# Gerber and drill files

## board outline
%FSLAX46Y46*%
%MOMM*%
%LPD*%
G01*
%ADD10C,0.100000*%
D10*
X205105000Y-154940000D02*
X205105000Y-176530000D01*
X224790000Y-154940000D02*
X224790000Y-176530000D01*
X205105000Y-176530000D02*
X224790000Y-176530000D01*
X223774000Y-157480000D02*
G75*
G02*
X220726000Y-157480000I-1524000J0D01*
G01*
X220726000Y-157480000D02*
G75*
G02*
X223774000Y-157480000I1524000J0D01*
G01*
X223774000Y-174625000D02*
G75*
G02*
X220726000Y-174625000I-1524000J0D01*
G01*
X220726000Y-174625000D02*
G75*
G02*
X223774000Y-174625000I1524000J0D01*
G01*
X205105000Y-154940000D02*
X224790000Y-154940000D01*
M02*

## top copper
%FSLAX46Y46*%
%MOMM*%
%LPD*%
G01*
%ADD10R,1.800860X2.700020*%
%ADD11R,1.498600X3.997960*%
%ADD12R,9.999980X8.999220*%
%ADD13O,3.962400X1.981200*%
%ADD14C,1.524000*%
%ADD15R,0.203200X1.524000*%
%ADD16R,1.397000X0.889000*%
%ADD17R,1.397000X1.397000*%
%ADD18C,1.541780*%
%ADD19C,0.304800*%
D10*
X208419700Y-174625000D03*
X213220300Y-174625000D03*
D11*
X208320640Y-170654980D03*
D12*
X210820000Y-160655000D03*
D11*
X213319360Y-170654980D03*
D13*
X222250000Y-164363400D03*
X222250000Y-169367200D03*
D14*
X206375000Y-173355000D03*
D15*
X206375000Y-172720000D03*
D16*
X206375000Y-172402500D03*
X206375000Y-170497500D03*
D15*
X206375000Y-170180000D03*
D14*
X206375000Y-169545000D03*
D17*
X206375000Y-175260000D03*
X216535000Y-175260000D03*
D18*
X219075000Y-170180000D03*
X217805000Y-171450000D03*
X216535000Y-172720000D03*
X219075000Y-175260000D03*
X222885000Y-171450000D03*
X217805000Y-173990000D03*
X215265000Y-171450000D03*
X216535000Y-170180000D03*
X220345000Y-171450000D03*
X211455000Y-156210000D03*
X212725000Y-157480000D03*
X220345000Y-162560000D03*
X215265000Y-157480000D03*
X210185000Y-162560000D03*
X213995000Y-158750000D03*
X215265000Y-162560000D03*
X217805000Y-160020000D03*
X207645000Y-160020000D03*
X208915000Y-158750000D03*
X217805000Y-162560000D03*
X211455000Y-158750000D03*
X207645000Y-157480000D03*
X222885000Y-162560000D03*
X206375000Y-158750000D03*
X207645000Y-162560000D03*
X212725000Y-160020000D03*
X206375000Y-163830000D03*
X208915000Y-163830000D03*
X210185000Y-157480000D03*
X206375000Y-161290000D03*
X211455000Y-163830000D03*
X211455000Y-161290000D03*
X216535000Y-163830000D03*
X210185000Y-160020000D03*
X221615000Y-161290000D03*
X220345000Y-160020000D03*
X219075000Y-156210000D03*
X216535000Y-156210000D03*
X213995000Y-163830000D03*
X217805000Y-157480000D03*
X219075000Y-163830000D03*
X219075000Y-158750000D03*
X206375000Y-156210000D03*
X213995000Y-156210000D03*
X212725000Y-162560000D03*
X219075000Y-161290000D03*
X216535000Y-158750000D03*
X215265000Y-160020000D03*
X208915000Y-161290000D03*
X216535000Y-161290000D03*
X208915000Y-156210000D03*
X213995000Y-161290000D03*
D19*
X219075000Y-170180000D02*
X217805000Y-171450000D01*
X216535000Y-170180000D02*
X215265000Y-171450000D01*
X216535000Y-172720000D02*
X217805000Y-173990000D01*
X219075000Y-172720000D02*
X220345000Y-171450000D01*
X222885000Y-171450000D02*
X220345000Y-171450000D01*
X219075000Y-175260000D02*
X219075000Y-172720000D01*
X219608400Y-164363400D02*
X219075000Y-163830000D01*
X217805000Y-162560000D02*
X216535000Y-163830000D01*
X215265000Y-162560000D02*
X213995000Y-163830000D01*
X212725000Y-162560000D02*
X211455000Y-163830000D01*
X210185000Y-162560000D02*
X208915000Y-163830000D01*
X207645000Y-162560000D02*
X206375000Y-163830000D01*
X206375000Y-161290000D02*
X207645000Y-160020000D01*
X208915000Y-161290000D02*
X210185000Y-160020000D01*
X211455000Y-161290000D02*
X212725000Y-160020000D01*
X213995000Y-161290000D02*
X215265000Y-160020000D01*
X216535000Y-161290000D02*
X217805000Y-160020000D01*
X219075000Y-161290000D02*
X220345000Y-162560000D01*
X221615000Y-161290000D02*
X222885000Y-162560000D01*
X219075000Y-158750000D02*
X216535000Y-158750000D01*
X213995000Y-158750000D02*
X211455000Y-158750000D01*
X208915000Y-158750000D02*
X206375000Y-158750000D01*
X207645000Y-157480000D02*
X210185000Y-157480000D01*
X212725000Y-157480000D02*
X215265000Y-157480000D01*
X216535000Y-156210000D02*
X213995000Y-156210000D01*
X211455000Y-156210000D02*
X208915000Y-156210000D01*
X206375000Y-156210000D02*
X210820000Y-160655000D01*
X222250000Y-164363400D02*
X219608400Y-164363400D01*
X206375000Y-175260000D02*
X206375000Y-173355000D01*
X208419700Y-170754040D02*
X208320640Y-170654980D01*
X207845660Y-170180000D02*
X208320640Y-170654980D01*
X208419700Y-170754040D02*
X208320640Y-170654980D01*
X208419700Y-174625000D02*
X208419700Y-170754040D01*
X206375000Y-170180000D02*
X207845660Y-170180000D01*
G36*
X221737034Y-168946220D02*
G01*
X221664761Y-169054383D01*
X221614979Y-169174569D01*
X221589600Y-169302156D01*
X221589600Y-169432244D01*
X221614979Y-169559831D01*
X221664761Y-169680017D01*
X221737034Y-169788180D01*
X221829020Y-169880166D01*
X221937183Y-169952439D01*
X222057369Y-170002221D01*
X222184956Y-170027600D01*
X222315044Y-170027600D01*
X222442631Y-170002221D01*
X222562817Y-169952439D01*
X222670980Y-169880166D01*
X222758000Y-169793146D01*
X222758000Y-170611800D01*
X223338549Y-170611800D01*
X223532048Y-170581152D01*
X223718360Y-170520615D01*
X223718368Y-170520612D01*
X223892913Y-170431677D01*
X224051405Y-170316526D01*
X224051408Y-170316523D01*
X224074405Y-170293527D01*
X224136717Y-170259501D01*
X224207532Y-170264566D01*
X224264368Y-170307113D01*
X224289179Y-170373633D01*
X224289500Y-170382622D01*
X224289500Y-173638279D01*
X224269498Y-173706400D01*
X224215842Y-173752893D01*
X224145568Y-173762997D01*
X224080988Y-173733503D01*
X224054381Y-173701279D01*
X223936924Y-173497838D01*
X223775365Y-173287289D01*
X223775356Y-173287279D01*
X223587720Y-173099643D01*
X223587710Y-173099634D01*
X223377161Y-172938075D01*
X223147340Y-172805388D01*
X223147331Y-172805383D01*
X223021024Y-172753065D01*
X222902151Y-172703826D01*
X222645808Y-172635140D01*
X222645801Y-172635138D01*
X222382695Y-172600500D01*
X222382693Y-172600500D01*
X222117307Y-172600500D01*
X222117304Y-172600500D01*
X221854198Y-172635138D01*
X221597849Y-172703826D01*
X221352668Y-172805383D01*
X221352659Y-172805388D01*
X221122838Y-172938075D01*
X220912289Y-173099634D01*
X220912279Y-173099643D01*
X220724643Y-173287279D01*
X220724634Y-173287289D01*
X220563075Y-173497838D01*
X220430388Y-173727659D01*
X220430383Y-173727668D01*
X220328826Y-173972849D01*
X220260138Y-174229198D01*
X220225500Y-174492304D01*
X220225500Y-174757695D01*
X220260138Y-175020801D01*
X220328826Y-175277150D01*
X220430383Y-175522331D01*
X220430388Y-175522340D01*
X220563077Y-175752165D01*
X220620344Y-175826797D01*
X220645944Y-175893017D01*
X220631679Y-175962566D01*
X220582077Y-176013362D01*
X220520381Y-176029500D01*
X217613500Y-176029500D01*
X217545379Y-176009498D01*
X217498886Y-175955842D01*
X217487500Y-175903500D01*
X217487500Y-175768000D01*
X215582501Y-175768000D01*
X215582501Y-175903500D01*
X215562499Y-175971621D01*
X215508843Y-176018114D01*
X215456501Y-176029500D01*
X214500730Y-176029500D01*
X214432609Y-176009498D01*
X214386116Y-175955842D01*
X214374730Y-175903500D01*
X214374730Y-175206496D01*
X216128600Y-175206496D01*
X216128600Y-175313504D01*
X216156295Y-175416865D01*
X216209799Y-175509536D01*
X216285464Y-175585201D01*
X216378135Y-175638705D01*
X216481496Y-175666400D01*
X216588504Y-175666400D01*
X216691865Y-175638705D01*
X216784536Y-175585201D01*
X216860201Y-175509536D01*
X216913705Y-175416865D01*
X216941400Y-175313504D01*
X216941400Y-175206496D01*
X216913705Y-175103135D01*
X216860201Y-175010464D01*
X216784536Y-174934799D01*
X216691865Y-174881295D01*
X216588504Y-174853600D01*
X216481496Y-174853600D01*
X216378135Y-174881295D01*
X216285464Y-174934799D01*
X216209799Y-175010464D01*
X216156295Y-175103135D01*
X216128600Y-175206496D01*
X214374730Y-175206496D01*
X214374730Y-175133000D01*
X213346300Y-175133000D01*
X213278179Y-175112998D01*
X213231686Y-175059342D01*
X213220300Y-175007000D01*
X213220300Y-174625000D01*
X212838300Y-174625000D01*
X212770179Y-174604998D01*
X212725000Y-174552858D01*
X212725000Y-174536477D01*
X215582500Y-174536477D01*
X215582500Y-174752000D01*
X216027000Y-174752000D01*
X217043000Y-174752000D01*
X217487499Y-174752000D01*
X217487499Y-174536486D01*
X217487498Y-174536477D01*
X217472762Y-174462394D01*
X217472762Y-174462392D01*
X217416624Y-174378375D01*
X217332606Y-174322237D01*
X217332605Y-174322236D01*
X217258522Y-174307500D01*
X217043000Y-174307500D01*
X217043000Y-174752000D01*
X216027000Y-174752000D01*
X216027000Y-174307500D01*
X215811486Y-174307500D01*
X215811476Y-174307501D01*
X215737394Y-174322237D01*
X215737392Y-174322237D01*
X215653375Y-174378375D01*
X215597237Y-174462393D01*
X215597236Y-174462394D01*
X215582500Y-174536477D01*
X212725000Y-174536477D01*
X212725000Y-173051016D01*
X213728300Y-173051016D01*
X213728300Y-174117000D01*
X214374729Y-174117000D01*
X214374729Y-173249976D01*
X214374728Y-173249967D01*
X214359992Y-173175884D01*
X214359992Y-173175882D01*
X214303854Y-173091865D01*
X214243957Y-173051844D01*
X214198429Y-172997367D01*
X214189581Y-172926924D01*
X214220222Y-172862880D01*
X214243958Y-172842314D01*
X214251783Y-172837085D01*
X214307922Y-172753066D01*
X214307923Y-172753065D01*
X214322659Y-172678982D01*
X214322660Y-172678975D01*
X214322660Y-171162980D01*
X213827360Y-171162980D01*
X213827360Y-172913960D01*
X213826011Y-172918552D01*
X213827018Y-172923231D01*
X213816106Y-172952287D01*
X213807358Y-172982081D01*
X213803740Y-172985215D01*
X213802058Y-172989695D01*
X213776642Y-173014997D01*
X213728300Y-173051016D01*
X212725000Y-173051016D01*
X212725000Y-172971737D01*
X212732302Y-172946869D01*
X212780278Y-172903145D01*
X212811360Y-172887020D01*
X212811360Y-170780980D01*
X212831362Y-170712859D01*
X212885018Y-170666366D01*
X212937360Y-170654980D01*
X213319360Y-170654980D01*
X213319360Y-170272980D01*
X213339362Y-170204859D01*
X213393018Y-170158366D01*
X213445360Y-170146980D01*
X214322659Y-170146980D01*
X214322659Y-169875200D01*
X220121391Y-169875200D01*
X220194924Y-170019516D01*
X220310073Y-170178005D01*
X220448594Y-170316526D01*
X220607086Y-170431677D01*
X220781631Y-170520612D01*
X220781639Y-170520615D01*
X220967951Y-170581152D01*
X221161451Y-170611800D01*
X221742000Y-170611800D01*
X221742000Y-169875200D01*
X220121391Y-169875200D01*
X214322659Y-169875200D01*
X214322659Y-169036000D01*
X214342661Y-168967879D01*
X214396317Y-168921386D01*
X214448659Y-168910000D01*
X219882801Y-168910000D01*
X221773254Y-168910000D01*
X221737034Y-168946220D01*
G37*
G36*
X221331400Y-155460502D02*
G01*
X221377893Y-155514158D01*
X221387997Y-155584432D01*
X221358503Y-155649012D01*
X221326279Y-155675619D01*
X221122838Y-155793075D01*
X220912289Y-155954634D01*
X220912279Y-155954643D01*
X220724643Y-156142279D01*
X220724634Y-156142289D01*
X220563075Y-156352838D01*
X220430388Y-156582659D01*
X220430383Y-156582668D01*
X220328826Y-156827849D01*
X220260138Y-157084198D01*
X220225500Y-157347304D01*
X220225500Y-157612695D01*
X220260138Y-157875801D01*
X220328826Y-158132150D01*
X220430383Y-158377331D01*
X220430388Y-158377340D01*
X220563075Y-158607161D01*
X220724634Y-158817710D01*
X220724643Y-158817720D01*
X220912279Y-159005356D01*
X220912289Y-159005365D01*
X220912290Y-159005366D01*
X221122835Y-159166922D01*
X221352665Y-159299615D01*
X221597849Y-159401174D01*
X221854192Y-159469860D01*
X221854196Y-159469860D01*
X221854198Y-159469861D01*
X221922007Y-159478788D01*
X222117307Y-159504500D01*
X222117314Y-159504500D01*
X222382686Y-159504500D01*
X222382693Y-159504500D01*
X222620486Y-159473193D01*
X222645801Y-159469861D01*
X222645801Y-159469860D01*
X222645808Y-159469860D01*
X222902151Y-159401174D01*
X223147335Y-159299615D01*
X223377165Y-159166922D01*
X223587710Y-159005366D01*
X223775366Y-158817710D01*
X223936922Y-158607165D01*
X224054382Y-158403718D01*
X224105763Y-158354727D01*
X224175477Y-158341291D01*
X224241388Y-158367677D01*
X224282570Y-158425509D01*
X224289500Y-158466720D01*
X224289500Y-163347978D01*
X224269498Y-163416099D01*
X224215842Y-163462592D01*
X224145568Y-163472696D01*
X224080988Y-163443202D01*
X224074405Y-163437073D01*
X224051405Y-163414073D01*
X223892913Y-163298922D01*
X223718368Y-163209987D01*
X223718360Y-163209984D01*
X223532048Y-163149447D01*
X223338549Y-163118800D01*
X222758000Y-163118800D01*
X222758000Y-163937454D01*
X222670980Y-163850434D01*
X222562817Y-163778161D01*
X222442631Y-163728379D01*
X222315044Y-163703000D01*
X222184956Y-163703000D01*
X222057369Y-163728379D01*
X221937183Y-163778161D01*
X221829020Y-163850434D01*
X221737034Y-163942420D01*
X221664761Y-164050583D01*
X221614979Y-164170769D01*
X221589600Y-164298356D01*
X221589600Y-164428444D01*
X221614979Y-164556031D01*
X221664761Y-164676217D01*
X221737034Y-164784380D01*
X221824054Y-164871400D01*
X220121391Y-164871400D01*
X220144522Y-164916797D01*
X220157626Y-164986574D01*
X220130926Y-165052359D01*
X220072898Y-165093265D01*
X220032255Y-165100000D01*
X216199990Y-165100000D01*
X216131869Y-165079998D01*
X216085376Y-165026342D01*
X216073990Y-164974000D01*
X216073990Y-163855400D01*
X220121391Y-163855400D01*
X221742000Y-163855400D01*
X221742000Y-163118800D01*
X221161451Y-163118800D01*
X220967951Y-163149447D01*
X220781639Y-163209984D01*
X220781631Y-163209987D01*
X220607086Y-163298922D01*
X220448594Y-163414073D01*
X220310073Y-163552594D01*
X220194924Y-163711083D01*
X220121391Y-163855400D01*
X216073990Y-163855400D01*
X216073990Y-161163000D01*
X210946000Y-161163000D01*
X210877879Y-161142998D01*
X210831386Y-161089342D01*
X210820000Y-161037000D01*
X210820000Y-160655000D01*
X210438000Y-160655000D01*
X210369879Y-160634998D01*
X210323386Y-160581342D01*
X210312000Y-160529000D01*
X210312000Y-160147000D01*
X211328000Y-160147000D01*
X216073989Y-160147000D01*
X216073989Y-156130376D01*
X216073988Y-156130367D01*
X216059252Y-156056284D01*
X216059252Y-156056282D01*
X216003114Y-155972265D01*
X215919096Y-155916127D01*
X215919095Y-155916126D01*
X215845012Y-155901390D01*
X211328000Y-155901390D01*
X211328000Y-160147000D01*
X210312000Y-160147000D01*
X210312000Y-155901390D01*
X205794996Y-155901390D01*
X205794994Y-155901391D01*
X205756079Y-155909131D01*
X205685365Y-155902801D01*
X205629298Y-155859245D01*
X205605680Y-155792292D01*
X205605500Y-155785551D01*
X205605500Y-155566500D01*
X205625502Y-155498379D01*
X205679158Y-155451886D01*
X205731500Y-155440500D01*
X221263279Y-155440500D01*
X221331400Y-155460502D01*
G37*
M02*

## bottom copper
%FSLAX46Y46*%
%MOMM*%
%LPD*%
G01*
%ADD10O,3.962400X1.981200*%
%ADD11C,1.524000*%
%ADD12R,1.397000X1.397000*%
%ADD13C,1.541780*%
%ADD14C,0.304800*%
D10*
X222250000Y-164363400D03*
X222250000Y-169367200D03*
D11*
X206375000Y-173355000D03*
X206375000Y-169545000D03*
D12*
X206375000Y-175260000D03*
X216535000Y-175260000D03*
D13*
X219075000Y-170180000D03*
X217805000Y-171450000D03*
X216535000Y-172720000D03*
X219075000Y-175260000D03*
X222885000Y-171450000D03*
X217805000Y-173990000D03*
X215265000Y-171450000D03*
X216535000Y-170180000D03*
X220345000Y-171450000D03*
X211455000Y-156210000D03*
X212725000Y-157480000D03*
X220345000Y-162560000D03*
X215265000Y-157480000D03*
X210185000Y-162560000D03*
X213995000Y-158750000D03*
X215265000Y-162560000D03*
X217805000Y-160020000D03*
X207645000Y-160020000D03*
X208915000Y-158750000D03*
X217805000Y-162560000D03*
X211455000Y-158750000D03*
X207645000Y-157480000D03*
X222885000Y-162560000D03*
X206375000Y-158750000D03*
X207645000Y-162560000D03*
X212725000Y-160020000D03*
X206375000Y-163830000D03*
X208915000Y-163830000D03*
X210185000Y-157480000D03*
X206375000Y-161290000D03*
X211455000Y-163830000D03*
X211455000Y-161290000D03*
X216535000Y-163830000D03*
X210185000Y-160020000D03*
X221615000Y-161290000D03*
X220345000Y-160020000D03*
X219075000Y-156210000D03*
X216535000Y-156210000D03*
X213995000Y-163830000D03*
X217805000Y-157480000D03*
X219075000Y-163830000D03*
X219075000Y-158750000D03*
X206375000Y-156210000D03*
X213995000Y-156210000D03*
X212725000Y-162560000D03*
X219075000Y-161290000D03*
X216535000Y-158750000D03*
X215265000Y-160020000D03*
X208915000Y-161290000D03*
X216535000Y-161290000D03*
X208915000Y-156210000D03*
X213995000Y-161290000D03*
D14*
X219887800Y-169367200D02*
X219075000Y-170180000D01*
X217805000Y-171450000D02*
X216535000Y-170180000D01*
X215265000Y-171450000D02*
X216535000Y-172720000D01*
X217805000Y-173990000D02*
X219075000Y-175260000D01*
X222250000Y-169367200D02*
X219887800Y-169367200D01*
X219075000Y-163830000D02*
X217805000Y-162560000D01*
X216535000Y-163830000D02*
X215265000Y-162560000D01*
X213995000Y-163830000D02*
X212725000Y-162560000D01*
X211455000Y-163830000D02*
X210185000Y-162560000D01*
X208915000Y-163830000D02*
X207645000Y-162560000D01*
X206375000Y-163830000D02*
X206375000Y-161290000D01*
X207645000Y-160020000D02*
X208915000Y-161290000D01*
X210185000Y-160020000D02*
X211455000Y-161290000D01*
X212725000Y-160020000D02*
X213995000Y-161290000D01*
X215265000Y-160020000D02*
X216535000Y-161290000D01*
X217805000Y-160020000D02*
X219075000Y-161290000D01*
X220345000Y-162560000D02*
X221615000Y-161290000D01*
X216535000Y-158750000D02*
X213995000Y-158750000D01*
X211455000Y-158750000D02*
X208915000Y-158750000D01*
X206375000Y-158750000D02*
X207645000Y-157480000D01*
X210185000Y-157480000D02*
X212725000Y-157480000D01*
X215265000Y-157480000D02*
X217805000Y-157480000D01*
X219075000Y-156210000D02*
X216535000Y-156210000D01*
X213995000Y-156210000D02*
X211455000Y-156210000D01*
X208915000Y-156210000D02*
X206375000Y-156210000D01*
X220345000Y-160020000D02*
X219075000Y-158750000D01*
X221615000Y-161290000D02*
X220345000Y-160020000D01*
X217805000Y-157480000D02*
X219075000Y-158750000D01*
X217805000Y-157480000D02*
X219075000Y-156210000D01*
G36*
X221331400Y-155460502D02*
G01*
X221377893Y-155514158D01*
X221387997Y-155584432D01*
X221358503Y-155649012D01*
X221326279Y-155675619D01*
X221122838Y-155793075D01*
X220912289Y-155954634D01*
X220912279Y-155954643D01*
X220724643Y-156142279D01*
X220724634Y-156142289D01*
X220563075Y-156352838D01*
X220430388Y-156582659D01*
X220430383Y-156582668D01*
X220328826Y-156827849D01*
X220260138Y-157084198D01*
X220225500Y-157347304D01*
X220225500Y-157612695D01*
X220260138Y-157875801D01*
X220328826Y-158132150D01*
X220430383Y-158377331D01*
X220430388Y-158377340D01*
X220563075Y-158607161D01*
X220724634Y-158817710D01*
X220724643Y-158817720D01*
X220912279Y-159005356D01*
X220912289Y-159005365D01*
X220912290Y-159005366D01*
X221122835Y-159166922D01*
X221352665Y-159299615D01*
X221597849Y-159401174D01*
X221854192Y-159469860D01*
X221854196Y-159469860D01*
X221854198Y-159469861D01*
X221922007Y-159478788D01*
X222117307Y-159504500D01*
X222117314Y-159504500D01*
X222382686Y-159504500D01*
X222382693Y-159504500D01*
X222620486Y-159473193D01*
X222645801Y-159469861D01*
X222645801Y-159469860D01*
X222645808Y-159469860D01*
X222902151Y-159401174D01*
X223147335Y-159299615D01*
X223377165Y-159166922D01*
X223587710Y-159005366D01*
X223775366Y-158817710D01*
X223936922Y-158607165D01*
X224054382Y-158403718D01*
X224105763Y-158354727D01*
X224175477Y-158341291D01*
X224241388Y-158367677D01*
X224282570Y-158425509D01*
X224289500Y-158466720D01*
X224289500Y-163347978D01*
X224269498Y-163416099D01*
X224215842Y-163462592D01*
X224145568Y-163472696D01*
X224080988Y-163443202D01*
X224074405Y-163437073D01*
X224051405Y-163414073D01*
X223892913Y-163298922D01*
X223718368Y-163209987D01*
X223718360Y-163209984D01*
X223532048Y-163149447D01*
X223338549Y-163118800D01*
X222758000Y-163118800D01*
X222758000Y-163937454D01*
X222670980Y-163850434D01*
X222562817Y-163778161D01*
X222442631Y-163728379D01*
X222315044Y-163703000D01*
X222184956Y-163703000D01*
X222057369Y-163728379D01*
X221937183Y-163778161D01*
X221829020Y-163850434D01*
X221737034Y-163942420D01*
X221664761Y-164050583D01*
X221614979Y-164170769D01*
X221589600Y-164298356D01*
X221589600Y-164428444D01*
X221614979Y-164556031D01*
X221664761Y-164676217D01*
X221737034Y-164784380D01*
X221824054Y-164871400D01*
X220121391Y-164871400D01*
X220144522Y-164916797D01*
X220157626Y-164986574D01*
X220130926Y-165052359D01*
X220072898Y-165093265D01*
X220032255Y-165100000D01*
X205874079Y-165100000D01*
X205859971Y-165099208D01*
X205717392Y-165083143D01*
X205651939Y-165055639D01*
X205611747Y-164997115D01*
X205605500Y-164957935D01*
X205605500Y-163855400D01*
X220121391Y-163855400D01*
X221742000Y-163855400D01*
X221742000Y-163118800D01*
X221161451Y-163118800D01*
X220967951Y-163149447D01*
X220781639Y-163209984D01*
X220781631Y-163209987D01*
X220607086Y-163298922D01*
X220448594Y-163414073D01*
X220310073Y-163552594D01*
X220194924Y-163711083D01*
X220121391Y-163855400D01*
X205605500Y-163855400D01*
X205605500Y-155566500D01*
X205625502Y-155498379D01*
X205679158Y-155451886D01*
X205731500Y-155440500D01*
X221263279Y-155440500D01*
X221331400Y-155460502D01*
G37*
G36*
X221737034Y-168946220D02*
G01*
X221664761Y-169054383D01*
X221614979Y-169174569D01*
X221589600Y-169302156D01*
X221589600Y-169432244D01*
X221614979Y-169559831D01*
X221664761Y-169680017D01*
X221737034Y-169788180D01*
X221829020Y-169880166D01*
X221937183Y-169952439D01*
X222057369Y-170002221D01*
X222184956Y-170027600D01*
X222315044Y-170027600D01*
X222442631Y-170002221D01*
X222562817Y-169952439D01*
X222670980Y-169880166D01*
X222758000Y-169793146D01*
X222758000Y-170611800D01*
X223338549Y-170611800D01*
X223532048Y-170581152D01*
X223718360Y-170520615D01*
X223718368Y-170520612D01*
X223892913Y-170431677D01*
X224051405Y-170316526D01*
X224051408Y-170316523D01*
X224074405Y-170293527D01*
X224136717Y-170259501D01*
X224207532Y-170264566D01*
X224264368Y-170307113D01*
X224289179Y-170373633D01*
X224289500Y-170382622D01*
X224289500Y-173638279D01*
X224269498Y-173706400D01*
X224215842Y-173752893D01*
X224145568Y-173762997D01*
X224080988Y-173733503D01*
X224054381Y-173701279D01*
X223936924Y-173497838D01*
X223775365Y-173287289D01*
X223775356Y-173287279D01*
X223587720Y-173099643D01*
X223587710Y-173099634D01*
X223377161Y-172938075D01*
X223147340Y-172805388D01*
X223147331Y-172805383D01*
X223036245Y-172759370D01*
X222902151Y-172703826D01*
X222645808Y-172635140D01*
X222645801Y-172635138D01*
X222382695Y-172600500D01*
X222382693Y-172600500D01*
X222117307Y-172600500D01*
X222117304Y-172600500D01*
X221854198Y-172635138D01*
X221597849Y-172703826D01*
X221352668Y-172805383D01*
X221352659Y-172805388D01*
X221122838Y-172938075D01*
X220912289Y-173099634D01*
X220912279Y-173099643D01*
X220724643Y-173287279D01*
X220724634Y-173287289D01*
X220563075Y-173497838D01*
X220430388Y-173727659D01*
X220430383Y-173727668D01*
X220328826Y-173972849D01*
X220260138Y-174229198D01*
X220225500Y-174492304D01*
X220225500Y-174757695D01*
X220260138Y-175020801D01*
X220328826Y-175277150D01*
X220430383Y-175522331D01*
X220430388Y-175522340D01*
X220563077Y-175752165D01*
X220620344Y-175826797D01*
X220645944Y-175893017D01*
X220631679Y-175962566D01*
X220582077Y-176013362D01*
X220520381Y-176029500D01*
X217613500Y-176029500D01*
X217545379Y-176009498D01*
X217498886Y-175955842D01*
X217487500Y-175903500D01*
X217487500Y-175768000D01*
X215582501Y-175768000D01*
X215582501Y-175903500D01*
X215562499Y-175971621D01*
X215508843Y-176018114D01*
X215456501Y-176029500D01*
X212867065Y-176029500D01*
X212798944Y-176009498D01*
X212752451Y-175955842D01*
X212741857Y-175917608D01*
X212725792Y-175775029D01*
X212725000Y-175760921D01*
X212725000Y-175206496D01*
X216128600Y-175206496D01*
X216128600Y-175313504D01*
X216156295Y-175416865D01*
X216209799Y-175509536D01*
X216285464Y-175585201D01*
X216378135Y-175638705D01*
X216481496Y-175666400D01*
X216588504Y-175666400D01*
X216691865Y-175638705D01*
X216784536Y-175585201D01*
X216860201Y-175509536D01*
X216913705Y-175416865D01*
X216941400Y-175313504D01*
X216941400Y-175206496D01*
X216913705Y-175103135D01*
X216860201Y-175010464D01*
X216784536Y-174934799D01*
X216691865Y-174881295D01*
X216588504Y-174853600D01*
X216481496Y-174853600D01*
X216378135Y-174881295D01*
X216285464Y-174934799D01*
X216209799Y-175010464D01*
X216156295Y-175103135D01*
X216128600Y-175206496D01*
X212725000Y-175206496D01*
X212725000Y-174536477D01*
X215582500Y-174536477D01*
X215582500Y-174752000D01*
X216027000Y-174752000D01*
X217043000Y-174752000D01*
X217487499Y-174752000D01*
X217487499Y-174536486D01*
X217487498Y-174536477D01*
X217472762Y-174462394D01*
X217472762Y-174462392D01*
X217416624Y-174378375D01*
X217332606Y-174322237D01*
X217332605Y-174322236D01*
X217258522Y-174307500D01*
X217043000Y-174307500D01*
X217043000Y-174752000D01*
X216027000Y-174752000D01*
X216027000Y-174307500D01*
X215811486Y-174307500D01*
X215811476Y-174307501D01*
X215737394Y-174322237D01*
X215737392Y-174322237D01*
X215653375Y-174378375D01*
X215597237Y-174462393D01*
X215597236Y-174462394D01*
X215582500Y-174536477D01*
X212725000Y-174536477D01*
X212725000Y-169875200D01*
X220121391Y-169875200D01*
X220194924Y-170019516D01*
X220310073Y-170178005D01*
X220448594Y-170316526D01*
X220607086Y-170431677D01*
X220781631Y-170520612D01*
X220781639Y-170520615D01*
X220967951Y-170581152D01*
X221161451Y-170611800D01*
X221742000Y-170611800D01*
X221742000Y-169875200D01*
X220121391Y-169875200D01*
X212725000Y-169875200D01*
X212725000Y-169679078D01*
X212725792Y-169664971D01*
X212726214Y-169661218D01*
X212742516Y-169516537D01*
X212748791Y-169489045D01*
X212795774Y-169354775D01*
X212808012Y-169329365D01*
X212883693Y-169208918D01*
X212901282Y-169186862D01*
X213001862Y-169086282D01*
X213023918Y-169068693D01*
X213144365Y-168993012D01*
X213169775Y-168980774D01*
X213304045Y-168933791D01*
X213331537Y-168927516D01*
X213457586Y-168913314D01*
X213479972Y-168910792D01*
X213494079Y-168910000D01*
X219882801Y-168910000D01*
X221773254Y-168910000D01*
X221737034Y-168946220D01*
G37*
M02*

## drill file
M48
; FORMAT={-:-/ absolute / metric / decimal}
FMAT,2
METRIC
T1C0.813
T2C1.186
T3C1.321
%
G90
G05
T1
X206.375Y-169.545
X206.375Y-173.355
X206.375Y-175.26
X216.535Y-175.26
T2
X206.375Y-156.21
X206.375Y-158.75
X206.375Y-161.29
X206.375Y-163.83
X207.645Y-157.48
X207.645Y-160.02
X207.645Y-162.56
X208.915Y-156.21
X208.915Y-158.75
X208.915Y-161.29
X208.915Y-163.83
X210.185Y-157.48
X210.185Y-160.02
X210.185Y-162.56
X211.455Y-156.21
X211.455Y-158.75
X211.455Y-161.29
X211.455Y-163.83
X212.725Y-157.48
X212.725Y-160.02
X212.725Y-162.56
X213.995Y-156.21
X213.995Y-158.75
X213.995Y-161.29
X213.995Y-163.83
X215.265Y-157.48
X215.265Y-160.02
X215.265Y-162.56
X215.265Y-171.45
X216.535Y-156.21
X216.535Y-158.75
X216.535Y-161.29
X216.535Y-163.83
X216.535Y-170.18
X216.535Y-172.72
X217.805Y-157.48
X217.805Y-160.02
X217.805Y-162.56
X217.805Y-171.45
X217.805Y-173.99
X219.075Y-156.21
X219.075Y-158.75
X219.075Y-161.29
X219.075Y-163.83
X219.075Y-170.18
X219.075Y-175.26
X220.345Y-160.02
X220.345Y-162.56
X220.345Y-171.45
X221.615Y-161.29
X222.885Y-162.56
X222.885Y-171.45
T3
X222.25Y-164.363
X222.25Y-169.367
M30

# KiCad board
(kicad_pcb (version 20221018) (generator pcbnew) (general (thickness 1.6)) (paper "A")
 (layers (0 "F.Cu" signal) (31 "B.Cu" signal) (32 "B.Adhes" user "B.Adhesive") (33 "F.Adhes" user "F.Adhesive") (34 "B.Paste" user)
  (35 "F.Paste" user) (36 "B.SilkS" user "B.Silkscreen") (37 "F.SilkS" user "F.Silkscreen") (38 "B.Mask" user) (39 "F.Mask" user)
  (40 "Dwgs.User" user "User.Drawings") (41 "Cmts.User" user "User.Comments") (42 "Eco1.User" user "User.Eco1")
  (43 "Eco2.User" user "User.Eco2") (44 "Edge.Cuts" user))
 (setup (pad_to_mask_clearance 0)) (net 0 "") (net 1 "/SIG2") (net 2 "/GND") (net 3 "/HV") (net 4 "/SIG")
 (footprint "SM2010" (layer "F.Cu") (at 210.82 174.625)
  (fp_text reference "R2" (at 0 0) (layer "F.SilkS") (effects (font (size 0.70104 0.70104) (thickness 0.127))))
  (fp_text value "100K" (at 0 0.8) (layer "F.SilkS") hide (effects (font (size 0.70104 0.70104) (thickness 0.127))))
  (pad "1" smd rect (at -2.4003 0) (size 1.80086 2.70002) (layers "F.Cu" "F.Paste" "F.Mask") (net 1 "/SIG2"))
  (pad "2" smd rect (at 2.4003 0) (size 1.80086 2.70002) (layers "F.Cu" "F.Paste" "F.Mask") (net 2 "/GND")))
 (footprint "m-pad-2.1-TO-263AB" (layer "F.Cu") (at 210.82 160.655)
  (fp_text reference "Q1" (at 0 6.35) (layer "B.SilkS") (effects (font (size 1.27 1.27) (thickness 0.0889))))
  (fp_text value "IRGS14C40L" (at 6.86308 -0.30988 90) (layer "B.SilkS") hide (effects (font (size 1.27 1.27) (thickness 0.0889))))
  (pad "1" smd rect (at -2.49936 9.99998) (size 1.4986 3.99796) (layers "F.Cu" "F.Paste" "F.Mask") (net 1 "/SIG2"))
  (pad "2" smd rect (at 0 0) (size 9.99998 8.99922) (layers "F.Cu" "F.Paste" "F.Mask") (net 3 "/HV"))
  (pad "3" smd rect (at 2.49936 9.99998) (size 1.4986 3.99796) (layers "F.Cu" "F.Paste" "F.Mask") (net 2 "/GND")))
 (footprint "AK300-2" (layer "F.Cu") (at 222.25 166.878 -90)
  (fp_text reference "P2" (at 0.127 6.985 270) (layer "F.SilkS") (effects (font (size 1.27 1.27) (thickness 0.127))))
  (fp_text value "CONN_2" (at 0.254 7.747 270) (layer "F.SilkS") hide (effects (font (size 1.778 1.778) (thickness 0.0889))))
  (pad "1" thru_hole oval (at -2.5146 0 270) (size 1.9812 3.9624) (drill 1.3208) (layers "*.Cu" "F.Paste" "F.SilkS" "F.Mask") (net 3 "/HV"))
  (pad "2" thru_hole oval (at 2.4892 0 270) (size 1.9812 3.9624) (drill 1.3208) (layers "*.Cu" "F.Paste" "F.SilkS" "F.Mask") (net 2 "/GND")))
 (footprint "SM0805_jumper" (layer "F.Cu") (at 206.375 171.45 90)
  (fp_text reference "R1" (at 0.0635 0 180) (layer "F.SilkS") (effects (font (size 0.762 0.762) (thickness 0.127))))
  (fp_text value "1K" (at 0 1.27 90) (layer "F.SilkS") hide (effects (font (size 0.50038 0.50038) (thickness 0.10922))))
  (pad "1" thru_hole circle (at -1.905 0 90) (size 1.524 1.524) (drill 0.8128) (layers "*.Cu" "*.Mask" "F.SilkS") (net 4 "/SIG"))
  (pad "1" smd rect (at -1.27 0 90) (size 1.524 0.2032) (layers "F.Cu" "F.Paste" "F.Mask") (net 4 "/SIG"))
  (pad "1" smd rect (at -0.9525 0 90) (size 0.889 1.397) (layers "F.Cu" "F.Paste" "F.Mask") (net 4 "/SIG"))
  (pad "2" smd rect (at 0.9525 0 90) (size 0.889 1.397) (layers "F.Cu" "F.Paste" "F.Mask") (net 1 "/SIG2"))
  (pad "2" smd rect (at 1.27 0 90) (size 1.524 0.2032) (layers "F.Cu" "F.Paste" "F.Mask") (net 1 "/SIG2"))
  (pad "2" thru_hole circle (at 1.905 0 90) (size 1.524 1.524) (drill 0.8128) (layers "*.Cu" "*.Mask" "F.SilkS") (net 1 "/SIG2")))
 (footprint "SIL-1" (layer "F.Cu") (at 206.375 175.26 180)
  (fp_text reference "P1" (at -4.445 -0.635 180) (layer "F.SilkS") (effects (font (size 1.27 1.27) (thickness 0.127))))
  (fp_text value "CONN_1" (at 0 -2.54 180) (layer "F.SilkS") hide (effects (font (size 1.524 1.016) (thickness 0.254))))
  (pad "1" thru_hole rect (at 0 0 180) (size 1.397 1.397) (drill 0.8128) (layers "*.Cu" "*.Mask" "F.SilkS") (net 4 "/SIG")))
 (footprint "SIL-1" (layer "F.Cu") (at 216.535 175.26)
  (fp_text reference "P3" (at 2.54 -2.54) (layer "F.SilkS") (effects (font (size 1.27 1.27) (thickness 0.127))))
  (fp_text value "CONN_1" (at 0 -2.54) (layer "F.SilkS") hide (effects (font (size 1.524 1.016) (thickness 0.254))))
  (pad "1" thru_hole rect (at 0 0) (size 1.397 1.397) (drill 0.8128) (layers "*.Cu" "*.Mask" "F.SilkS") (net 2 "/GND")))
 (gr_line (start 205.105 154.94) (end 205.105 176.53) (stroke (width 0.1) (type solid)) (layer "Edge.Cuts"))
 (gr_line (start 224.79 154.94) (end 224.79 176.53) (stroke (width 0.1) (type solid)) (layer "Edge.Cuts"))
 (gr_line (start 205.105 176.53) (end 224.79 176.53) (stroke (width 0.1) (type solid)) (layer "Edge.Cuts"))
 (gr_circle (center 222.25 157.48) (end 223.774 157.48) (stroke (width 0.1) (type solid)) (fill none) (layer "Edge.Cuts"))
 (gr_circle (center 222.25 174.625) (end 223.774 174.625) (stroke (width 0.1) (type solid)) (fill none) (layer "Edge.Cuts"))
 (gr_line (start 205.105 154.94) (end 224.79 154.94) (stroke (width 0.1) (type solid)) (layer "Edge.Cuts"))
 (segment (start 219.075 170.18) (end 217.805 171.45) (width 0.3048) (layer "F.Cu") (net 2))
 (segment (start 216.535 170.18) (end 215.265 171.45) (width 0.3048) (layer "F.Cu") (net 2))
 (segment (start 216.535 172.72) (end 217.805 173.99) (width 0.3048) (layer "F.Cu") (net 2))
 (segment (start 219.075 172.72) (end 220.345 171.45) (width 0.3048) (layer "F.Cu") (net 2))
 (segment (start 222.885 171.45) (end 220.345 171.45) (width 0.3048) (layer "F.Cu") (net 2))
 (segment (start 219.075 175.26) (end 219.075 172.72) (width 0.3048) (layer "F.Cu") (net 2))
 (via (at 219.075 170.18) (size 1.54178) (drill 1.18618) (layers "F.Cu" "B.Cu") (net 2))
 (via (at 217.805 171.45) (size 1.54178) (drill 1.18618) (layers "F.Cu" "B.Cu") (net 2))
 (via (at 216.535 172.72) (size 1.54178) (drill 1.18618) (layers "F.Cu" "B.Cu") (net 2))
 (via (at 219.075 175.26) (size 1.54178) (drill 1.18618) (layers "F.Cu" "B.Cu") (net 2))
 (via (at 222.885 171.45) (size 1.54178) (drill 1.18618) (layers "F.Cu" "B.Cu") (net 2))
 (via (at 217.805 173.99) (size 1.54178) (drill 1.18618) (layers "F.Cu" "B.Cu") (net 2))
 (via (at 215.265 171.45) (size 1.54178) (drill 1.18618) (layers "F.Cu" "B.Cu") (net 2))
 (via (at 216.535 170.18) (size 1.54178) (drill 1.18618) (layers "F.Cu" "B.Cu") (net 2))
 (via (at 220.345 171.45) (size 1.54178) (drill 1.18618) (layers "F.Cu" "B.Cu") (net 2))
 (segment (start 219.8878 169.3672) (end 219.075 170.18) (width 0.3048) (layer "B.Cu") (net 2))
 (segment (start 217.805 171.45) (end 216.535 170.18) (width 0.3048) (layer "B.Cu") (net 2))
 (segment (start 215.265 171.45) (end 216.535 172.72) (width 0.3048) (layer "B.Cu") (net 2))
 (segment (start 217.805 173.99) (end 219.075 175.26) (width 0.3048) (layer "B.Cu") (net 2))
 (segment (start 222.25 169.3672) (end 219.8878 169.3672) (width 0.3048) (layer "B.Cu") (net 2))
 (segment (start 219.6084 164.3634) (end 219.075 163.83) (width 0.3048) (layer "F.Cu") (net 3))
 (segment (start 217.805 162.56) (end 216.535 163.83) (width 0.3048) (layer "F.Cu") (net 3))
 (segment (start 215.265 162.56) (end 213.995 163.83) (width 0.3048) (layer "F.Cu") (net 3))
 (segment (start 212.725 162.56) (end 211.455 163.83) (width 0.3048) (layer "F.Cu") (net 3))
 (segment (start 210.185 162.56) (end 208.915 163.83) (width 0.3048) (layer "F.Cu") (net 3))
 (segment (start 207.645 162.56) (end 206.375 163.83) (width 0.3048) (layer "F.Cu") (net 3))
 (segment (start 206.375 161.29) (end 207.645 160.02) (width 0.3048) (layer "F.Cu") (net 3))
 (segment (start 208.915 161.29) (end 210.185 160.02) (width 0.3048) (layer "F.Cu") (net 3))
 (segment (start 211.455 161.29) (end 212.725 160.02) (width 0.3048) (layer "F.Cu") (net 3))
 (segment (start 213.995 161.29) (end 215.265 160.02) (width 0.3048) (layer "F.Cu") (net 3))
 (segment (start 216.535 161.29) (end 217.805 160.02) (width 0.3048) (layer "F.Cu") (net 3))
 (segment (start 219.075 161.29) (end 220.345 162.56) (width 0.3048) (layer "F.Cu") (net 3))
 (segment (start 221.615 161.29) (end 222.885 162.56) (width 0.3048) (layer "F.Cu") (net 3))
 (segment (start 219.075 158.75) (end 216.535 158.75) (width 0.3048) (layer "F.Cu") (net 3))
 (segment (start 213.995 158.75) (end 211.455 158.75) (width 0.3048) (layer "F.Cu") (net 3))
 (segment (start 208.915 158.75) (end 206.375 158.75) (width 0.3048) (layer "F.Cu") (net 3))
 (segment (start 207.645 157.48) (end 210.185 157.48) (width 0.3048) (layer "F.Cu") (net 3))
 (segment (start 212.725 157.48) (end 215.265 157.48) (width 0.3048) (layer "F.Cu") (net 3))
 (segment (start 216.535 156.21) (end 213.995 156.21) (width 0.3048) (layer "F.Cu") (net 3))
 (segment (start 211.455 156.21) (end 208.915 156.21) (width 0.3048) (layer "F.Cu") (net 3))
 (segment (start 206.375 156.21) (end 210.82 160.655) (width 0.3048) (layer "F.Cu") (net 3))
 (segment (start 222.25 164.3634) (end 219.6084 164.3634) (width 0.3048) (layer "F.Cu") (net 3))
 (via (at 211.455 156.21) (size 1.54178) (drill 1.18618) (layers "F.Cu" "B.Cu") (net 3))
 (via (at 212.725 157.48) (size 1.54178) (drill 1.18618) (layers "F.Cu" "B.Cu") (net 3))
 (via (at 220.345 162.56) (size 1.54178) (drill 1.18618) (layers "F.Cu" "B.Cu") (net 3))
 (via (at 215.265 157.48) (size 1.54178) (drill 1.18618) (layers "F.Cu" "B.Cu") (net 3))
 (via (at 210.185 162.56) (size 1.54178) (drill 1.18618) (layers "F.Cu" "B.Cu") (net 3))
 (via (at 213.995 158.75) (size 1.54178) (drill 1.18618) (layers "F.Cu" "B.Cu") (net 3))
 (via (at 215.265 162.56) (size 1.54178) (drill 1.18618) (layers "F.Cu" "B.Cu") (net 3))
 (via (at 217.805 160.02) (size 1.54178) (drill 1.18618) (layers "F.Cu" "B.Cu") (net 3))
 (via (at 207.645 160.02) (size 1.54178) (drill 1.18618) (layers "F.Cu" "B.Cu") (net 3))
 (via (at 208.915 158.75) (size 1.54178) (drill 1.18618) (layers "F.Cu" "B.Cu") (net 3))
 (via (at 217.805 162.56) (size 1.54178) (drill 1.18618) (layers "F.Cu" "B.Cu") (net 3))
 (via (at 211.455 158.75) (size 1.54178) (drill 1.18618) (layers "F.Cu" "B.Cu") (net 3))
 (via (at 207.645 157.48) (size 1.54178) (drill 1.18618) (layers "F.Cu" "B.Cu") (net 3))
 (via (at 222.885 162.56) (size 1.54178) (drill 1.18618) (layers "F.Cu" "B.Cu") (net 3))
 (via (at 206.375 158.75) (size 1.54178) (drill 1.18618) (layers "F.Cu" "B.Cu") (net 3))
 (via (at 207.645 162.56) (size 1.54178) (drill 1.18618) (layers "F.Cu" "B.Cu") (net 3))
 (via (at 212.725 160.02) (size 1.54178) (drill 1.18618) (layers "F.Cu" "B.Cu") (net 3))
 (via (at 206.375 163.83) (size 1.54178) (drill 1.18618) (layers "F.Cu" "B.Cu") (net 3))
 (via (at 208.915 163.83) (size 1.54178) (drill 1.18618) (layers "F.Cu" "B.Cu") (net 3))
 (via (at 210.185 157.48) (size 1.54178) (drill 1.18618) (layers "F.Cu" "B.Cu") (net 3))
 (via (at 206.375 161.29) (size 1.54178) (drill 1.18618) (layers "F.Cu" "B.Cu") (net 3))
 (via (at 211.455 163.83) (size 1.54178) (drill 1.18618) (layers "F.Cu" "B.Cu") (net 3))
 (via (at 211.455 161.29) (size 1.54178) (drill 1.18618) (layers "F.Cu" "B.Cu") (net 3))
 (via (at 216.535 163.83) (size 1.54178) (drill 1.18618) (layers "F.Cu" "B.Cu") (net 3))
 (via (at 210.185 160.02) (size 1.54178) (drill 1.18618) (layers "F.Cu" "B.Cu") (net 3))
 (via (at 221.615 161.29) (size 1.54178) (drill 1.18618) (layers "F.Cu" "B.Cu") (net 3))
 (via (at 220.345 160.02) (size 1.54178) (drill 1.18618) (layers "F.Cu" "B.Cu") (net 3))
 (via (at 219.075 156.21) (size 1.54178) (drill 1.18618) (layers "F.Cu" "B.Cu") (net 3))
 (via (at 216.535 156.21) (size 1.54178) (drill 1.18618) (layers "F.Cu" "B.Cu") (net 3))
 (via (at 213.995 163.83) (size 1.54178) (drill 1.18618) (layers "F.Cu" "B.Cu") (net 3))
 (via (at 217.805 157.48) (size 1.54178) (drill 1.18618) (layers "F.Cu" "B.Cu") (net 3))
 (via (at 219.075 163.83) (size 1.54178) (drill 1.18618) (layers "F.Cu" "B.Cu") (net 3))
 (via (at 219.075 158.75) (size 1.54178) (drill 1.18618) (layers "F.Cu" "B.Cu") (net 3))
 (via (at 206.375 156.21) (size 1.54178) (drill 1.18618) (layers "F.Cu" "B.Cu") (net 3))
 (via (at 213.995 156.21) (size 1.54178) (drill 1.18618) (layers "F.Cu" "B.Cu") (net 3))
 (via (at 212.725 162.56) (size 1.54178) (drill 1.18618) (layers "F.Cu" "B.Cu") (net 3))
 (via (at 219.075 161.29) (size 1.54178) (drill 1.18618) (layers "F.Cu" "B.Cu") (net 3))
 (via (at 216.535 158.75) (size 1.54178) (drill 1.18618) (layers "F.Cu" "B.Cu") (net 3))
 (via (at 215.265 160.02) (size 1.54178) (drill 1.18618) (layers "F.Cu" "B.Cu") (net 3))
 (via (at 208.915 161.29) (size 1.54178) (drill 1.18618) (layers "F.Cu" "B.Cu") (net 3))
 (via (at 216.535 161.29) (size 1.54178) (drill 1.18618) (layers "F.Cu" "B.Cu") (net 3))
 (via (at 208.915 156.21) (size 1.54178) (drill 1.18618) (layers "F.Cu" "B.Cu") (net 3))
 (via (at 213.995 161.29) (size 1.54178) (drill 1.18618) (layers "F.Cu" "B.Cu") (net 3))
 (segment (start 219.075 163.83) (end 217.805 162.56) (width 0.3048) (layer "B.Cu") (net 3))
 (segment (start 216.535 163.83) (end 215.265 162.56) (width 0.3048) (layer "B.Cu") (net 3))
 (segment (start 213.995 163.83) (end 212.725 162.56) (width 0.3048) (layer "B.Cu") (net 3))
 (segment (start 211.455 163.83) (end 210.185 162.56) (width 0.3048) (layer "B.Cu") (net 3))
 (segment (start 208.915 163.83) (end 207.645 162.56) (width 0.3048) (layer "B.Cu") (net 3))
 (segment (start 206.375 163.83) (end 206.375 161.29) (width 0.3048) (layer "B.Cu") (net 3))
 (segment (start 207.645 160.02) (end 208.915 161.29) (width 0.3048) (layer "B.Cu") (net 3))
 (segment (start 210.185 160.02) (end 211.455 161.29) (width 0.3048) (layer "B.Cu") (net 3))
 (segment (start 212.725 160.02) (end 213.995 161.29) (width 0.3048) (layer "B.Cu") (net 3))
 (segment (start 215.265 160.02) (end 216.535 161.29) (width 0.3048) (layer "B.Cu") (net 3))
 (segment (start 217.805 160.02) (end 219.075 161.29) (width 0.3048) (layer "B.Cu") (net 3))
 (segment (start 220.345 162.56) (end 221.615 161.29) (width 0.3048) (layer "B.Cu") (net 3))
 (segment (start 216.535 158.75) (end 213.995 158.75) (width 0.3048) (layer "B.Cu") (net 3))
 (segment (start 211.455 158.75) (end 208.915 158.75) (width 0.3048) (layer "B.Cu") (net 3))
 (segment (start 206.375 158.75) (end 207.645 157.48) (width 0.3048) (layer "B.Cu") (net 3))
 (segment (start 210.185 157.48) (end 212.725 157.48) (width 0.3048) (layer "B.Cu") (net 3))
 (segment (start 215.265 157.48) (end 217.805 157.48) (width 0.3048) (layer "B.Cu") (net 3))
 (segment (start 219.075 156.21) (end 216.535 156.21) (width 0.3048) (layer "B.Cu") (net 3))
 (segment (start 213.995 156.21) (end 211.455 156.21) (width 0.3048) (layer "B.Cu") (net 3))
 (segment (start 208.915 156.21) (end 206.375 156.21) (width 0.3048) (layer "B.Cu") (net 3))
 (segment (start 220.345 160.02) (end 219.075 158.75) (width 0.3048) (layer "B.Cu") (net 3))
 (segment (start 221.615 161.29) (end 220.345 160.02) (width 0.3048) (layer "B.Cu") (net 3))
 (segment (start 217.805 157.48) (end 219.075 158.75) (width 0.3048) (layer "B.Cu") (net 3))
 (segment (start 217.805 157.48) (end 219.075 156.21) (width 0.3048) (layer "B.Cu") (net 3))
 (segment (start 206.375 175.26) (end 206.375 173.355) (width 0.3048) (layer "F.Cu") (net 4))
 (segment (start 208.4197 170.75404) (end 208.32064 170.65498) (width 0.3048) (layer "F.Cu") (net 1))
 (segment (start 207.84566 170.18) (end 208.32064 170.65498) (width 0.3048) (layer "F.Cu") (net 1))
 (segment (start 208.4197 170.75404) (end 208.32064 170.65498) (width 0.3048) (layer "F.Cu") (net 1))
 (segment (start 208.4197 174.625) (end 208.4197 170.75404) (width 0.3048) (layer "F.Cu") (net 1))
 (segment (start 206.375 170.18) (end 207.84566 170.18) (width 0.3048) (layer "F.Cu") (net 1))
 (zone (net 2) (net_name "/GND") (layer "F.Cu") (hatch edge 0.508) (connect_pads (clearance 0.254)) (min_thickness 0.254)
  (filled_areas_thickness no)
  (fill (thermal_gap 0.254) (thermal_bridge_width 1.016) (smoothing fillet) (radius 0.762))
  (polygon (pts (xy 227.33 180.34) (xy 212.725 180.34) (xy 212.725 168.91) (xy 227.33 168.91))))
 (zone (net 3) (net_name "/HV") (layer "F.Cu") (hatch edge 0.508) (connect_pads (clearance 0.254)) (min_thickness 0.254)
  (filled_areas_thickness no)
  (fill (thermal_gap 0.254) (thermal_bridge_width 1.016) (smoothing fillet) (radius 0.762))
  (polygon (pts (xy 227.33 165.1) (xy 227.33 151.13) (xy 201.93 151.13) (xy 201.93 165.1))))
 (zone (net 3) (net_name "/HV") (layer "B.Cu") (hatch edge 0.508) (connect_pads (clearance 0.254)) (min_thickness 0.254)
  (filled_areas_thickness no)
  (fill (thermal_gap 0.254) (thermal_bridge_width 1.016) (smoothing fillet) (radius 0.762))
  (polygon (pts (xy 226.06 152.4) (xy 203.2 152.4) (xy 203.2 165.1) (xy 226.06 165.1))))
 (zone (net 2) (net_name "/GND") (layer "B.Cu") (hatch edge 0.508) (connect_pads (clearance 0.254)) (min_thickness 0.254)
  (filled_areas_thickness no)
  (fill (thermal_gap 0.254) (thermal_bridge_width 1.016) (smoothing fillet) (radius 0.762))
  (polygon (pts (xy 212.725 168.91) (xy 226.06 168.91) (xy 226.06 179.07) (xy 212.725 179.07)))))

